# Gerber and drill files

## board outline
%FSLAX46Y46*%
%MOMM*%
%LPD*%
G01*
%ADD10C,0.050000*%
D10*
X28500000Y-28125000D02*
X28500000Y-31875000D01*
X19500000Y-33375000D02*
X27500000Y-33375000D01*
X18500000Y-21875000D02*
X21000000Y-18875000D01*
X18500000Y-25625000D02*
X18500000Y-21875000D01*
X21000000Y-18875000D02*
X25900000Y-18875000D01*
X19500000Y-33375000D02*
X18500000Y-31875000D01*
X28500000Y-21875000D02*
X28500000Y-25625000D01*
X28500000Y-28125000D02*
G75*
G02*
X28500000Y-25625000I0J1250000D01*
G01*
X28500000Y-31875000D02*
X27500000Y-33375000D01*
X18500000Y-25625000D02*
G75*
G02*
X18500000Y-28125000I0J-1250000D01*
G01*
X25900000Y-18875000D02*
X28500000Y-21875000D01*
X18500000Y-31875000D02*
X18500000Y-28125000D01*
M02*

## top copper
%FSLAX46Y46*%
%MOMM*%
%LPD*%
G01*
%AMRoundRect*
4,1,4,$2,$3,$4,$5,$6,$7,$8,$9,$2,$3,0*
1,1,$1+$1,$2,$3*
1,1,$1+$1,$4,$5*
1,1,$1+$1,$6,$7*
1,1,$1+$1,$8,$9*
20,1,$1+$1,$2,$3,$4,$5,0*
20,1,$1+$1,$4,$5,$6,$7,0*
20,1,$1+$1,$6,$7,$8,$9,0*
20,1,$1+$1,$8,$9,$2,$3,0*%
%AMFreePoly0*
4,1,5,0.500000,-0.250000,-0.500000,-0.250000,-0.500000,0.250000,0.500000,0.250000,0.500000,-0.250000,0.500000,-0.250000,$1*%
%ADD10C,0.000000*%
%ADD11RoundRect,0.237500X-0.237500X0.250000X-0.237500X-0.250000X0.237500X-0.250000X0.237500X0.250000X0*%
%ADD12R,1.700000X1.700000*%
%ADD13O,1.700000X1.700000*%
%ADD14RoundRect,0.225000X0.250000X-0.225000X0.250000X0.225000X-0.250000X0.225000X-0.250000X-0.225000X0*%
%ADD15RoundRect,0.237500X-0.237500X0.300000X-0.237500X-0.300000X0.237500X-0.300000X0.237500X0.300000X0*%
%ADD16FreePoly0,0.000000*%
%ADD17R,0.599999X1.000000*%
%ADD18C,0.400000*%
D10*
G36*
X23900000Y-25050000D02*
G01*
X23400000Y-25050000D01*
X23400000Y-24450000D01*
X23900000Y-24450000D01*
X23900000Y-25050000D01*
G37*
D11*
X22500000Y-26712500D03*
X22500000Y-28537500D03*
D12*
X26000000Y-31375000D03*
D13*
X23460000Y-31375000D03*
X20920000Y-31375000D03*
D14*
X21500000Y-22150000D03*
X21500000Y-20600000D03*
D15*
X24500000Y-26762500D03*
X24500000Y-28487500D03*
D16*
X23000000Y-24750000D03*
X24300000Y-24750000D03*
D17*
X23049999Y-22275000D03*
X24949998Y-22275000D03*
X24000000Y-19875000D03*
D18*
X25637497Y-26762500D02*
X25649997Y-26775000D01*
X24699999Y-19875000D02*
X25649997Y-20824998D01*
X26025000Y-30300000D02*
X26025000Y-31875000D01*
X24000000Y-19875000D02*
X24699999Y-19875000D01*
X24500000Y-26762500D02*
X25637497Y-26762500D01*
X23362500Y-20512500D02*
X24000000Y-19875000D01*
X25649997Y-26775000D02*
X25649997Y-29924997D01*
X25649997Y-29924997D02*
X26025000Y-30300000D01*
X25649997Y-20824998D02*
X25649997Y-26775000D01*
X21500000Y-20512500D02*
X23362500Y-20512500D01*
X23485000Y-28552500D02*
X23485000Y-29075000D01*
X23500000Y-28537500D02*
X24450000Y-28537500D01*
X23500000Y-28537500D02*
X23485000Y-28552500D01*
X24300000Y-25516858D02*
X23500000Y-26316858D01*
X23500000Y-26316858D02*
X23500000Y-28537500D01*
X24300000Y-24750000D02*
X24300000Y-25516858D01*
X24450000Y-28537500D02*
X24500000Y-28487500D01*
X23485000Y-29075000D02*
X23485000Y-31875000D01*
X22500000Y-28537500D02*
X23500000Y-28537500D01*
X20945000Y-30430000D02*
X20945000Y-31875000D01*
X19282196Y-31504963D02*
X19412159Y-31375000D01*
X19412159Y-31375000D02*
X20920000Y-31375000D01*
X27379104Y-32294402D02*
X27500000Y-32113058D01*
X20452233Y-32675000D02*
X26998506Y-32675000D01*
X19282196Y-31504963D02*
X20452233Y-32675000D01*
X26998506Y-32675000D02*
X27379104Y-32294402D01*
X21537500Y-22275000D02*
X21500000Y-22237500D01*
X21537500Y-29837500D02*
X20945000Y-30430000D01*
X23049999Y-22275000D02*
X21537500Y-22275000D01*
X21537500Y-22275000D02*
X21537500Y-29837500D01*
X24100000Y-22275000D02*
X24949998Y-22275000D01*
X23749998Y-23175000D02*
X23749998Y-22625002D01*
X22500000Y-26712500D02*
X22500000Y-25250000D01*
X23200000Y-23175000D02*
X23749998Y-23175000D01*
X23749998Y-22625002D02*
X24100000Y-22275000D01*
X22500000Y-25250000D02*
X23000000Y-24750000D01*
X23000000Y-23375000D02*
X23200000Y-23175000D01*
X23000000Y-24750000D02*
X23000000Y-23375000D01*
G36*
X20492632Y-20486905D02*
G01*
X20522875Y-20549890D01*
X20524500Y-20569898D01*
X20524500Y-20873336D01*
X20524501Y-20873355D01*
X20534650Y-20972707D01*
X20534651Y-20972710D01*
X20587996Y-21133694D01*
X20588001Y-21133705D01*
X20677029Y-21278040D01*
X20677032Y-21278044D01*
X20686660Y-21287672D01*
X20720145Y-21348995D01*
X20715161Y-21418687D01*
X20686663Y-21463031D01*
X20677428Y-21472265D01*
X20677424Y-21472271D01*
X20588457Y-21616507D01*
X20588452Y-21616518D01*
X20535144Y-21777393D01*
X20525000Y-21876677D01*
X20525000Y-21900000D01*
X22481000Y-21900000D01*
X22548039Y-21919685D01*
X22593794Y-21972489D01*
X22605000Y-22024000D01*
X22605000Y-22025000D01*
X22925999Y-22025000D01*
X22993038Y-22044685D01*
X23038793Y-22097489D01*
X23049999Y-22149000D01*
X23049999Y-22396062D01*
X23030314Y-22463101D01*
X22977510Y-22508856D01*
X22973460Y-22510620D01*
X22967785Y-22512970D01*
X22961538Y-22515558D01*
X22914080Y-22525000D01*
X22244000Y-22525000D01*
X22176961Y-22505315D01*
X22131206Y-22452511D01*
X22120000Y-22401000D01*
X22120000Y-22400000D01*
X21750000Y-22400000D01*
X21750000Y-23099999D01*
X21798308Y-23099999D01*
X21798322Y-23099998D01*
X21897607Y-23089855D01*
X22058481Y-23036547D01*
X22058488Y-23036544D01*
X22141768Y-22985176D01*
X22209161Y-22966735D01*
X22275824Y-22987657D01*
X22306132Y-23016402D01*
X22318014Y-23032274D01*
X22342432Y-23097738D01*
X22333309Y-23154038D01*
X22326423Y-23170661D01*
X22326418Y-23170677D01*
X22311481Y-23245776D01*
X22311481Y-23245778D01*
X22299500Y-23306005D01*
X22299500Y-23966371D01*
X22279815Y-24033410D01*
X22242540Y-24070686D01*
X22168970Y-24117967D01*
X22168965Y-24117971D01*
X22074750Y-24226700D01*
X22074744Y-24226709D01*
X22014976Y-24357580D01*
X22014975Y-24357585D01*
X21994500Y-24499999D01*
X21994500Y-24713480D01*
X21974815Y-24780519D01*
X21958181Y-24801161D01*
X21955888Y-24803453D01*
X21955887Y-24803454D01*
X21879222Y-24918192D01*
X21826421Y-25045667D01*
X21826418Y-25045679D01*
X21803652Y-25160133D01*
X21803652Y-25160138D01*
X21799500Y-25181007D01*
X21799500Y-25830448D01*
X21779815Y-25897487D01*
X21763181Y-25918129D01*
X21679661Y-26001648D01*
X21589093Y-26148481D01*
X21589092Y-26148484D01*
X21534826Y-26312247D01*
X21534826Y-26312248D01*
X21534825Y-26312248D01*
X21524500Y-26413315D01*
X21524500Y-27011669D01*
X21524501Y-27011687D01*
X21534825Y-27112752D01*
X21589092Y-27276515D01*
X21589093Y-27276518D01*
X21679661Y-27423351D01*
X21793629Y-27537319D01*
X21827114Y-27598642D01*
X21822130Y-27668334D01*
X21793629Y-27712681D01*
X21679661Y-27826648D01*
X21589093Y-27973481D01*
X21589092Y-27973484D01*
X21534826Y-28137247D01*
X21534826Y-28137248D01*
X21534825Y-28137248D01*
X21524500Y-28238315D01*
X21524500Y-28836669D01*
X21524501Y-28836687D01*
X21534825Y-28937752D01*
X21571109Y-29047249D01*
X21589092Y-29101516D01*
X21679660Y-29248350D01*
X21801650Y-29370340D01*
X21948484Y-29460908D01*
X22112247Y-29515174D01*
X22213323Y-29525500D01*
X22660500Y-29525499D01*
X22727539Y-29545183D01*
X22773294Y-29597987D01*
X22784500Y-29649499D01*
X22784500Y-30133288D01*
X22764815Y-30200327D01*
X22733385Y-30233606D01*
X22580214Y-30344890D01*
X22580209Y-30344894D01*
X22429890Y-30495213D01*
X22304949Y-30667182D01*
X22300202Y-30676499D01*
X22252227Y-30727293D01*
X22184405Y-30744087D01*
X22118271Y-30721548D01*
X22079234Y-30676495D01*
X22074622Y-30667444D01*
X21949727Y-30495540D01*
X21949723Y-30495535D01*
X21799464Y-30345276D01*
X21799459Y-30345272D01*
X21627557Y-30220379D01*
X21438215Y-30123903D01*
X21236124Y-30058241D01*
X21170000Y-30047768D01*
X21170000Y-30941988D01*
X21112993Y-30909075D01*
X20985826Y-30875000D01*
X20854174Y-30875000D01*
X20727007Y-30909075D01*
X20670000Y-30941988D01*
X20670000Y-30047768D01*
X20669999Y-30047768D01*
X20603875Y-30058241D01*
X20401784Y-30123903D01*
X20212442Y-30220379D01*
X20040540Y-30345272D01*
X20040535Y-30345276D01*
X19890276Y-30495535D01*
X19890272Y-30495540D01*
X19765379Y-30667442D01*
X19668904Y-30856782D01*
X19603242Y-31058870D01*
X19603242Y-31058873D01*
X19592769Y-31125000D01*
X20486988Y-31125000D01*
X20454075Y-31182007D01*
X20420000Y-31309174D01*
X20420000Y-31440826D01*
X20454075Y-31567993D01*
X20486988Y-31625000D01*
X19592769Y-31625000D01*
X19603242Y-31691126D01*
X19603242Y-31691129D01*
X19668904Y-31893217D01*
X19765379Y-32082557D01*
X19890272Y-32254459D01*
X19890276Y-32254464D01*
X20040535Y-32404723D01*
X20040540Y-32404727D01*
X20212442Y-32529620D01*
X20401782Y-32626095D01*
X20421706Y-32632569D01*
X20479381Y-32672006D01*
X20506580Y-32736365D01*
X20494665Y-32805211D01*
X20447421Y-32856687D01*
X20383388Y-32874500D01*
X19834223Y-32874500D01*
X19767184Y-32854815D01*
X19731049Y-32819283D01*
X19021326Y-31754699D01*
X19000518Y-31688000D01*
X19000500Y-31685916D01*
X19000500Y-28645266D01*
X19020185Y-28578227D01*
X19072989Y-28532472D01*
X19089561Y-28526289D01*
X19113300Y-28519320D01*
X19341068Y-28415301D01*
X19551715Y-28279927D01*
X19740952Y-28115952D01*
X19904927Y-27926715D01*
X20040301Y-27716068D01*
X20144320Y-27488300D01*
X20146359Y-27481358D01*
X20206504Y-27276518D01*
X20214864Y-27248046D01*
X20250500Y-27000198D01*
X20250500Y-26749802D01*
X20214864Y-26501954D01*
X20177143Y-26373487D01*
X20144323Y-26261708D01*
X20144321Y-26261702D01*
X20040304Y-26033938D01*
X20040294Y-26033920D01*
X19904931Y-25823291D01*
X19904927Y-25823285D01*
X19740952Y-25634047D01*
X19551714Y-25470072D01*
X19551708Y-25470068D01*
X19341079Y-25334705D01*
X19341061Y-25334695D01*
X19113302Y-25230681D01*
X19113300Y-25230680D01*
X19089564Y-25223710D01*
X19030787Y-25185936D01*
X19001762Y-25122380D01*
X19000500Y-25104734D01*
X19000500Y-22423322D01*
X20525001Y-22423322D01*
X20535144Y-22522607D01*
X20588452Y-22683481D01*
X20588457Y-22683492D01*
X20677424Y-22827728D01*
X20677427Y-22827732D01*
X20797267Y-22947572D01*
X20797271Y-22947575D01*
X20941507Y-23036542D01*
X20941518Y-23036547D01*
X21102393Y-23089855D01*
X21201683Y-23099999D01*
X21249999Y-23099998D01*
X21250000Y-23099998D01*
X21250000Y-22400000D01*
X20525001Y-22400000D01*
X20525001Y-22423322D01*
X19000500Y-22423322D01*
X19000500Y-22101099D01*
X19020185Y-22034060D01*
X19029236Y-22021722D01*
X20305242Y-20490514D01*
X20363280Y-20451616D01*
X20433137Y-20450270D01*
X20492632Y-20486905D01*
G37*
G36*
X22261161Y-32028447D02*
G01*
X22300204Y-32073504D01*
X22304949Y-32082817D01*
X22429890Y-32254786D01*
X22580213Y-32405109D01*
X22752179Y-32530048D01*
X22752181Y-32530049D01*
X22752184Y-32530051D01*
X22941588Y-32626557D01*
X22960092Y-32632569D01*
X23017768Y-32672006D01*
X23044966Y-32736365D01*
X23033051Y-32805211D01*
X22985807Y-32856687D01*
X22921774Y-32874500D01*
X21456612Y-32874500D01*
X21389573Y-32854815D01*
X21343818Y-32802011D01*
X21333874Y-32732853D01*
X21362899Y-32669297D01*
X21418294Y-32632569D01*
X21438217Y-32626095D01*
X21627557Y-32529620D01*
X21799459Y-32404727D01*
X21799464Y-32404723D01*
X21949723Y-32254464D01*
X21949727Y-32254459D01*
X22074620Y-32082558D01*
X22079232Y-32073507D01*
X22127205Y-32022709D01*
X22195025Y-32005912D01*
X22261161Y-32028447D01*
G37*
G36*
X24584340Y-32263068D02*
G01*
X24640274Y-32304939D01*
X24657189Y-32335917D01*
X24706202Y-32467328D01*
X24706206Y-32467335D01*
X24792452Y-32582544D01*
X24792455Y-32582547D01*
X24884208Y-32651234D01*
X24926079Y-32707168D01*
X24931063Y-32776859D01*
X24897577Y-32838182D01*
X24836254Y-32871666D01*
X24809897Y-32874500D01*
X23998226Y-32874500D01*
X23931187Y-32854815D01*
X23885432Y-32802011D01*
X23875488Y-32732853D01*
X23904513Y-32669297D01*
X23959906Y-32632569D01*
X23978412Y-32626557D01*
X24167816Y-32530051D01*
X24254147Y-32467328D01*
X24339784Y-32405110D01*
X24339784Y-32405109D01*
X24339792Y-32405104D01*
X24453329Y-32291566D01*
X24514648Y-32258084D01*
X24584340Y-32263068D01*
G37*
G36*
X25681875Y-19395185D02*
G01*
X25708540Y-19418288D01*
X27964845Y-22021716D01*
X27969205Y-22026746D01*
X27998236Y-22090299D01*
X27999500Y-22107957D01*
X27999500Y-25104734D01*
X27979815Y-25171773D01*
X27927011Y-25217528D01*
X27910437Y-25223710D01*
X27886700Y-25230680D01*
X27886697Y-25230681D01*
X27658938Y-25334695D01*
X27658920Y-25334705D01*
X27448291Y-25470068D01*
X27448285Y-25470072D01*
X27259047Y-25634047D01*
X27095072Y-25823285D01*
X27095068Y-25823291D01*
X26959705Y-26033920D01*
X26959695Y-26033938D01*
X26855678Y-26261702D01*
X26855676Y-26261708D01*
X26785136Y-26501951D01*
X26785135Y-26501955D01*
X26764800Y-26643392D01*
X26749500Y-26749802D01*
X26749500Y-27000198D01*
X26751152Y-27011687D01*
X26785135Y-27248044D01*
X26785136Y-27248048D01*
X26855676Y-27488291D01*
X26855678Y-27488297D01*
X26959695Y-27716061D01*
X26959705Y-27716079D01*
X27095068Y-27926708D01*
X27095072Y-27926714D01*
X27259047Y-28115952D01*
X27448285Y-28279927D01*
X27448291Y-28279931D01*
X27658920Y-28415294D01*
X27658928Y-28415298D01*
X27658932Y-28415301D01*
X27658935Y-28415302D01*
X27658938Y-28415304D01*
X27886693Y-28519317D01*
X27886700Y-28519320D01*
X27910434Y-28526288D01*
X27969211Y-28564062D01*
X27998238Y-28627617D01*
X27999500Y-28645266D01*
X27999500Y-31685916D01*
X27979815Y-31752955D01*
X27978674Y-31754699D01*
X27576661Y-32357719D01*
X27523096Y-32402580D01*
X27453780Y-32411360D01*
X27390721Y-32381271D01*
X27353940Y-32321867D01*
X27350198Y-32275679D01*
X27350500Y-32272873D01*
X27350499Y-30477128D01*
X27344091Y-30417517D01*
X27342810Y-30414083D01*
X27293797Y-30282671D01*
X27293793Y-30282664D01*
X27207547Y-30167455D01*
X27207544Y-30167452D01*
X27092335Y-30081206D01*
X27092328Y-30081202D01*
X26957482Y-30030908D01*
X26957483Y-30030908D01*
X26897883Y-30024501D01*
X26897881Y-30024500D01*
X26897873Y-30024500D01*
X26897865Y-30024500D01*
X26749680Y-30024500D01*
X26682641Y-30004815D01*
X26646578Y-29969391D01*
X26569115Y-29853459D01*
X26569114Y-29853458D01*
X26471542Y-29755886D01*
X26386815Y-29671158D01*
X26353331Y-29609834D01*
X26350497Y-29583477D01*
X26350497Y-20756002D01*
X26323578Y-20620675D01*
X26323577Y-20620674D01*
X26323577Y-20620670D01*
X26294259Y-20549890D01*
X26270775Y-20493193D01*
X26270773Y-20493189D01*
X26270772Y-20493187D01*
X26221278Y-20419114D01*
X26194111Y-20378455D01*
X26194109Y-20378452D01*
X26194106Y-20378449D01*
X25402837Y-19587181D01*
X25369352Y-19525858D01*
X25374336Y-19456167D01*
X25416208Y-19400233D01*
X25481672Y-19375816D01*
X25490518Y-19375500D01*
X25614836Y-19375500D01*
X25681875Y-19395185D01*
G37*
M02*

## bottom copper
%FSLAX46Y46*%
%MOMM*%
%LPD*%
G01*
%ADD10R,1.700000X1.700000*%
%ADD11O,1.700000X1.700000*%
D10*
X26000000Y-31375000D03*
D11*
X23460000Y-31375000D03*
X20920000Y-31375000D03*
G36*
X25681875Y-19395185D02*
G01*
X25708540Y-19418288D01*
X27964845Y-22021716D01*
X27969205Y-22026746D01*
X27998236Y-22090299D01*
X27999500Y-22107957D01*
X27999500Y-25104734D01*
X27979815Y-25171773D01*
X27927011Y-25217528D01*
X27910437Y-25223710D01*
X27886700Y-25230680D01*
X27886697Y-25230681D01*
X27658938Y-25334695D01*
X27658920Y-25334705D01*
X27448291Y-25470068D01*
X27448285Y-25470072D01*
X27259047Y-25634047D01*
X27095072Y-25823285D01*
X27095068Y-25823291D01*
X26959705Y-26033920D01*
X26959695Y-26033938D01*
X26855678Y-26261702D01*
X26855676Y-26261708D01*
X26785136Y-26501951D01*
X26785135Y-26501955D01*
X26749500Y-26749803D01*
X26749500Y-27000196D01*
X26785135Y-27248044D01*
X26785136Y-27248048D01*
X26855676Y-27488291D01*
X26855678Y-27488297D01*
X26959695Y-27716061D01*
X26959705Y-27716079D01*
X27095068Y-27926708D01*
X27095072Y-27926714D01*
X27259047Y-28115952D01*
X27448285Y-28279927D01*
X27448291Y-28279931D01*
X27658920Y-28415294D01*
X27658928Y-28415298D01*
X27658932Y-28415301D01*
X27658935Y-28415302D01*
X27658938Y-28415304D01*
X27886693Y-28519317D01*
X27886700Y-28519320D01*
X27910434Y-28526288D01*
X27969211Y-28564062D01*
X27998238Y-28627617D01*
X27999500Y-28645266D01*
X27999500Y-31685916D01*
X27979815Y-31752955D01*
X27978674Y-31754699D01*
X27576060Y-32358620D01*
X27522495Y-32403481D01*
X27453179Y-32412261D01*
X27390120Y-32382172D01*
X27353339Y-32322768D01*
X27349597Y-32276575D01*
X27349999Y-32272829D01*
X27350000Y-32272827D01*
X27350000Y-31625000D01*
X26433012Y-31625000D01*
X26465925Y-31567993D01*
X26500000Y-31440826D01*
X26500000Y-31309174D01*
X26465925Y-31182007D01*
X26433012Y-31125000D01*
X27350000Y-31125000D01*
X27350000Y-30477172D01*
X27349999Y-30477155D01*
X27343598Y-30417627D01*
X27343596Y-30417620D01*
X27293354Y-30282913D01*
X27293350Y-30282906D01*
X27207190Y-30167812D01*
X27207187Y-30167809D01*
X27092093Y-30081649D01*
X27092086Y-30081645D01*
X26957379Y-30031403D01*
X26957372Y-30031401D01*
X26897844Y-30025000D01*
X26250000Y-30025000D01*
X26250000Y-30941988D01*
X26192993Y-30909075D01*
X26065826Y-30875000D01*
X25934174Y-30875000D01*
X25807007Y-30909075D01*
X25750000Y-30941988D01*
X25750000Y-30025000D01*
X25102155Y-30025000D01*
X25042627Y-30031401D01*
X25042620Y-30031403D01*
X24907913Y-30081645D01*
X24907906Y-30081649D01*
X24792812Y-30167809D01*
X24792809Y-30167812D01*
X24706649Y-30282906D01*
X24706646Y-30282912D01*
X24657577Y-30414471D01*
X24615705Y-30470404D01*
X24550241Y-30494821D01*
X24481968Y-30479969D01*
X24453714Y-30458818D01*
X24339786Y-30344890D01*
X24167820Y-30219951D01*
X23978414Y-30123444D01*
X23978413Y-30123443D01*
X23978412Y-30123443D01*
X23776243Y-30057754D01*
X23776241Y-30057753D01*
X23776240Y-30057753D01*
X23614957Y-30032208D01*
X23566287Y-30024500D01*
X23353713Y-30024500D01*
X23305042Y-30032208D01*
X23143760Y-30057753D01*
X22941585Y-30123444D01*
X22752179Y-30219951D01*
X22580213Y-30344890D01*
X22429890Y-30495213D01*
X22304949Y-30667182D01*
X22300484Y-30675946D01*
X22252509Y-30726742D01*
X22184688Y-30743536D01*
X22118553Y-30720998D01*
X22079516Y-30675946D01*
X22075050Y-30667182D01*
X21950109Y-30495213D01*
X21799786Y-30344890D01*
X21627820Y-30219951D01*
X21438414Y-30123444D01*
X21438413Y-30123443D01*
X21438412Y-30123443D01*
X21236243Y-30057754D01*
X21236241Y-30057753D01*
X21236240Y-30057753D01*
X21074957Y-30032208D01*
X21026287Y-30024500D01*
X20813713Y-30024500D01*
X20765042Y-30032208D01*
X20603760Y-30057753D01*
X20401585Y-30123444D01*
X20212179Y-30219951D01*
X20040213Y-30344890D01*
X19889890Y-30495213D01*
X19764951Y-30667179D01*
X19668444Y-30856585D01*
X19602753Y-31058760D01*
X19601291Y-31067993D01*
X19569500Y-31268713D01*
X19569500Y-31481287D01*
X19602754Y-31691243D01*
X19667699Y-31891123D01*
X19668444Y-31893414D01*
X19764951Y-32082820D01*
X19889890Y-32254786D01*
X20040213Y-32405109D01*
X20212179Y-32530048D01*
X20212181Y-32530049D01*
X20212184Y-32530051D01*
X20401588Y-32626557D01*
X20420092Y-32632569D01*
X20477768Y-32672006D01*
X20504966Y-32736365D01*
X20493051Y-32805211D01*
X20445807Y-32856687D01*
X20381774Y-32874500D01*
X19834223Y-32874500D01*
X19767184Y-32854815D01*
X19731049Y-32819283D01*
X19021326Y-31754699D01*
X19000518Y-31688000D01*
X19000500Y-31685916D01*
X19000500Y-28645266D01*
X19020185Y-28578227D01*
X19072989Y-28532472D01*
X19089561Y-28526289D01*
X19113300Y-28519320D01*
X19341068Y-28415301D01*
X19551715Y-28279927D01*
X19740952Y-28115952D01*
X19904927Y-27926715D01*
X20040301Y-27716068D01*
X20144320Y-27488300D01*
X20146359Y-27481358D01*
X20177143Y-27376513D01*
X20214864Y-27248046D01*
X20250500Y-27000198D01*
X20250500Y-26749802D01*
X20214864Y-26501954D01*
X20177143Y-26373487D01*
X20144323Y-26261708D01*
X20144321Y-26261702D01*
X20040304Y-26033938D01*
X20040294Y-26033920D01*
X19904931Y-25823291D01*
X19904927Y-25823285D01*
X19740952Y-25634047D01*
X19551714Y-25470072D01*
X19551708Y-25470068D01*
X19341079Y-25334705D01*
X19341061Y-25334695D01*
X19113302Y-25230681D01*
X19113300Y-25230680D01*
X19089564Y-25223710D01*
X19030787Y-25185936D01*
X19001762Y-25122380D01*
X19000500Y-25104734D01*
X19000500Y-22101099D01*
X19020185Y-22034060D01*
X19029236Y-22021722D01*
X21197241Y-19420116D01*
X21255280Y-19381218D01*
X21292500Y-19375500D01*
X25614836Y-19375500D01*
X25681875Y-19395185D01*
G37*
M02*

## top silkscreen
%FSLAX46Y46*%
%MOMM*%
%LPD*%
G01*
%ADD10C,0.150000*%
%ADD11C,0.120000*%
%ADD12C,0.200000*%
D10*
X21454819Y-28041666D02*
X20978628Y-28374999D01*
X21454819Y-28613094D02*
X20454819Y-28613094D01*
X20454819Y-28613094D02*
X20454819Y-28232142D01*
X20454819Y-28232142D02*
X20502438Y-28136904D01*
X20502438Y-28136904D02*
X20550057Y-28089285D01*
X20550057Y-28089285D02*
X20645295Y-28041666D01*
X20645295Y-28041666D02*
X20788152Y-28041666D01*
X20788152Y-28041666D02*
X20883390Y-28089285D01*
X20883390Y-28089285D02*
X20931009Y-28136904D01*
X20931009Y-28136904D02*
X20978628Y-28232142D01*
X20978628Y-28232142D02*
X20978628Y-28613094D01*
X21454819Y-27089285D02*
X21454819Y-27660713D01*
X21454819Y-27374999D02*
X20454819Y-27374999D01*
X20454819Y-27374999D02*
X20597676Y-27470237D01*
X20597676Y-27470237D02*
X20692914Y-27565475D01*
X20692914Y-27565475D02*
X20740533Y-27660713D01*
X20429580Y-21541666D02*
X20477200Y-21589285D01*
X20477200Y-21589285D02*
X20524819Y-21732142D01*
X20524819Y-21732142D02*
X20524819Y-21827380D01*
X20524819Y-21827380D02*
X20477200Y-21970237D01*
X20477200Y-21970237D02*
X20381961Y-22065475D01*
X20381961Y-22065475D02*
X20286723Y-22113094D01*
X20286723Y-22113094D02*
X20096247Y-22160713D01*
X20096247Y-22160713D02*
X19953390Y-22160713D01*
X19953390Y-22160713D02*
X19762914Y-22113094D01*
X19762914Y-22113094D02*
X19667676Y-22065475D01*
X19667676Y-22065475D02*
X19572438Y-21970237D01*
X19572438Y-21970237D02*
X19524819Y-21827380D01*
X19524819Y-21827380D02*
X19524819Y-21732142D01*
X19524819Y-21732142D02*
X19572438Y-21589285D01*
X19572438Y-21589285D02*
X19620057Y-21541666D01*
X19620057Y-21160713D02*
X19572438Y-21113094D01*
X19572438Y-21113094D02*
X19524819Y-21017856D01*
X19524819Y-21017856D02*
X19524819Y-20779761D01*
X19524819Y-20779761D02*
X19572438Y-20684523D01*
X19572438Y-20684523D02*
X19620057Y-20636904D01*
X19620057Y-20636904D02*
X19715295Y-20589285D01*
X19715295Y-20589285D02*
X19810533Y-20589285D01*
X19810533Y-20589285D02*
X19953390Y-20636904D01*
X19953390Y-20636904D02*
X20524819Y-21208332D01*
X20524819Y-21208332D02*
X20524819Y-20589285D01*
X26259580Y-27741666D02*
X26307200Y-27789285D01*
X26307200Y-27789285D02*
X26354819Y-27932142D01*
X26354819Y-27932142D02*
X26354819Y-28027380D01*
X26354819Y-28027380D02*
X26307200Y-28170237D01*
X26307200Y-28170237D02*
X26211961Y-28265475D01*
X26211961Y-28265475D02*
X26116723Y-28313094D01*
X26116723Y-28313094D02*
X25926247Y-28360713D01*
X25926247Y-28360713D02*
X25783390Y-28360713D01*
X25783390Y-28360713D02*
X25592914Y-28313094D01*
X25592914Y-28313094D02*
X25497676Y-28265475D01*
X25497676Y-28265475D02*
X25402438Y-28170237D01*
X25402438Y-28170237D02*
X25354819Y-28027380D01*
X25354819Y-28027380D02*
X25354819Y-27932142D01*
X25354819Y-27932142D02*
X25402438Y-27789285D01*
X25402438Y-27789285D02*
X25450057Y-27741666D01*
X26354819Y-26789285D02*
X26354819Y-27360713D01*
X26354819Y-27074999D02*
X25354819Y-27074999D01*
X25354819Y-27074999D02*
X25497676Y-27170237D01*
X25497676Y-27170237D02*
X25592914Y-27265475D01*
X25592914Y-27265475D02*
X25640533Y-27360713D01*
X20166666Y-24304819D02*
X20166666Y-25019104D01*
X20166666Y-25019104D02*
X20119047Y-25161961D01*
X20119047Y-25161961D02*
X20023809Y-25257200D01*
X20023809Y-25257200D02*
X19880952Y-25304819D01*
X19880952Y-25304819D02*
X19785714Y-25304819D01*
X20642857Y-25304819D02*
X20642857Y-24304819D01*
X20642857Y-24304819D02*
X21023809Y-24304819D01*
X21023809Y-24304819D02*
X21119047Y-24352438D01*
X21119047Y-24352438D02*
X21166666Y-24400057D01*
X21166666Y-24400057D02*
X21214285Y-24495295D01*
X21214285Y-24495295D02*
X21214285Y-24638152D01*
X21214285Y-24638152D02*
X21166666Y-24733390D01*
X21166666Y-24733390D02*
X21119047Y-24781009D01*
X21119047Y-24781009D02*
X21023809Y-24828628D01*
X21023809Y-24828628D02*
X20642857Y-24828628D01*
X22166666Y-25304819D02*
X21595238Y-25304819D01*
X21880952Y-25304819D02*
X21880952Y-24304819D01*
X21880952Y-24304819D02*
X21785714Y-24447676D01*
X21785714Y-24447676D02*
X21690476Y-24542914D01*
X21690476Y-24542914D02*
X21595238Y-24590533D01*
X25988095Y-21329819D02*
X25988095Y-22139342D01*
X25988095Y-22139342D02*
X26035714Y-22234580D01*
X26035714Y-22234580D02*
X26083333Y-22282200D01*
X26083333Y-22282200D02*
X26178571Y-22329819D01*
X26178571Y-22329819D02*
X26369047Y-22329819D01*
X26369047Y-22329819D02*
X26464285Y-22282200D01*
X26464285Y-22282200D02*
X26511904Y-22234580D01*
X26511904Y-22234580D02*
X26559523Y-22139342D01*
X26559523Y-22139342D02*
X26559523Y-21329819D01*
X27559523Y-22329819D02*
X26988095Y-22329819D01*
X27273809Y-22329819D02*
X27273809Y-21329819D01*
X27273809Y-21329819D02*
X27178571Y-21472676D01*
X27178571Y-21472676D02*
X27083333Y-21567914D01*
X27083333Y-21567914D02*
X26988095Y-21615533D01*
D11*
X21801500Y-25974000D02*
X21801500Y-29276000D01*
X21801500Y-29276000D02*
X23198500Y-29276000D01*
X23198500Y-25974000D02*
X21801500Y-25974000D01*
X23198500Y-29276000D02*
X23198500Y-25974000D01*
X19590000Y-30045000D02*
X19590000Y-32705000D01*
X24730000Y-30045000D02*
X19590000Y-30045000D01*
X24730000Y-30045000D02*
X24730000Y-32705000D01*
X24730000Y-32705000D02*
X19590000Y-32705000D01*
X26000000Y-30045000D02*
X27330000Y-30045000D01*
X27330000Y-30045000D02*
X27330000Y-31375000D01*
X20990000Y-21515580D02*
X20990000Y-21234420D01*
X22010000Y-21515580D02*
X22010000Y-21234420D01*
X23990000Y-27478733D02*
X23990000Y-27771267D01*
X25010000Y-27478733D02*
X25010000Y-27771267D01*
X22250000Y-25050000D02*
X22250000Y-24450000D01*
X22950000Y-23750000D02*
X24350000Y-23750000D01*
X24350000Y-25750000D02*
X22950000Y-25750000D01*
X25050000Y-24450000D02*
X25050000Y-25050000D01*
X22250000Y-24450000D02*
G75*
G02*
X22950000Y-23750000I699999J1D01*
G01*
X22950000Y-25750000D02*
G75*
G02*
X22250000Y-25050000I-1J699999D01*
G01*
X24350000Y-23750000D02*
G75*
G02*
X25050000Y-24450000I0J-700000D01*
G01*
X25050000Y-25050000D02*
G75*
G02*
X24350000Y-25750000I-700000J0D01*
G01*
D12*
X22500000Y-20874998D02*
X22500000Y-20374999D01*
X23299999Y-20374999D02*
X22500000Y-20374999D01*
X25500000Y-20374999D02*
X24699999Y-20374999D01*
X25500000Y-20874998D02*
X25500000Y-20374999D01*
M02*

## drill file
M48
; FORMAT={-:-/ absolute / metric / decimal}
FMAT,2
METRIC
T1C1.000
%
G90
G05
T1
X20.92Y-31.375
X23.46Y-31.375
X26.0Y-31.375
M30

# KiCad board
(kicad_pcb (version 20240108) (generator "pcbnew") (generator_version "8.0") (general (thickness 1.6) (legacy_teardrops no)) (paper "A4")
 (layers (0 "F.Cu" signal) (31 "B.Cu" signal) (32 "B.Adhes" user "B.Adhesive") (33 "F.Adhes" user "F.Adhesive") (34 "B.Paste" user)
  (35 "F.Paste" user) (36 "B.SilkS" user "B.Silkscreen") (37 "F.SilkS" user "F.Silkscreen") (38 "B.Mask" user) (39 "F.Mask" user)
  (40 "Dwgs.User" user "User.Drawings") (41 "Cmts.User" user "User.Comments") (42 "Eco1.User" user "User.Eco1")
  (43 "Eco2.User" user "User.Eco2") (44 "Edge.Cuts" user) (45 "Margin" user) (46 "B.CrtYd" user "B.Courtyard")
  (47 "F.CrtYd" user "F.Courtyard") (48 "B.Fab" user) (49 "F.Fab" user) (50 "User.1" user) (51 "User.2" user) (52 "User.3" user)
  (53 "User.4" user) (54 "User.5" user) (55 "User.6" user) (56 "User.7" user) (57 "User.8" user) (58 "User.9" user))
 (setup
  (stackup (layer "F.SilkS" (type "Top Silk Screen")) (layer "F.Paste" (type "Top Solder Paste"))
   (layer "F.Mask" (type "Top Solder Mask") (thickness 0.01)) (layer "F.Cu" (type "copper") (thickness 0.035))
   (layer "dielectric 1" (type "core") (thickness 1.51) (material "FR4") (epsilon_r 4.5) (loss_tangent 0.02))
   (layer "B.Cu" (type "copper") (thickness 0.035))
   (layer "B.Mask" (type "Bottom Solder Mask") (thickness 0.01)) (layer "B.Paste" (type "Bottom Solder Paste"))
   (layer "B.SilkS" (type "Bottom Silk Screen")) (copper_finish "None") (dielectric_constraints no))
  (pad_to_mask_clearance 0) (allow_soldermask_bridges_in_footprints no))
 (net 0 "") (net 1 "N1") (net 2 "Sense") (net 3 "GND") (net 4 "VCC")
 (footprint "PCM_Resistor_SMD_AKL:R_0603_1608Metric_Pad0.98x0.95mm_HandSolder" (layer "F.Cu") (at 22.5 27.625 -90)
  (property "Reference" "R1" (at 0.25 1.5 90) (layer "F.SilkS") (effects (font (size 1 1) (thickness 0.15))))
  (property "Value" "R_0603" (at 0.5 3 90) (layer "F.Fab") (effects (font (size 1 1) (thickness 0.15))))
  (fp_line (start -1.651 0.6985) (end 1.651 0.6985) (stroke (width 0.12) (type solid)) (layer "F.SilkS"))
  (fp_line (start 1.651 0.6985) (end 1.651 -0.6985) (stroke (width 0.12) (type solid)) (layer "F.SilkS"))
  (fp_line (start -1.651 -0.6985) (end -1.651 0.6985) (stroke (width 0.12) (type solid)) (layer "F.SilkS"))
  (fp_line (start 1.651 -0.6985) (end -1.651 -0.6985) (stroke (width 0.12) (type solid)) (layer "F.SilkS"))
  (pad "1" smd roundrect (at -0.9125 0 270) (size 0.975 0.95) (layers "F.Cu" "F.Paste" "F.Mask") (roundrect_rratio 0.25) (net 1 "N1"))
  (pad "2" smd roundrect (at 0.9125 0 270) (size 0.975 0.95) (layers "F.Cu" "F.Paste" "F.Mask") (roundrect_rratio 0.25) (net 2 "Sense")))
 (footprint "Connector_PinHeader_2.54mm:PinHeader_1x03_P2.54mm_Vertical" (layer "F.Cu") (at 26 31.375 -90)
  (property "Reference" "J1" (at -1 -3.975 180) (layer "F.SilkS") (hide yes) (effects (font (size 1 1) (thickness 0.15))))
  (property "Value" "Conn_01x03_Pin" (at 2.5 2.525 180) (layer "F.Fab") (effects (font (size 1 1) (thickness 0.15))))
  (fp_line (start -1.33 6.41) (end 1.33 6.41) (stroke (width 0.12) (type solid)) (layer "F.SilkS"))
  (fp_line (start -1.33 1.27) (end -1.33 6.41) (stroke (width 0.12) (type solid)) (layer "F.SilkS"))
  (fp_line (start -1.33 1.27) (end 1.33 1.27) (stroke (width 0.12) (type solid)) (layer "F.SilkS"))
  (fp_line (start 1.33 1.27) (end 1.33 6.41) (stroke (width 0.12) (type solid)) (layer "F.SilkS"))
  (fp_line (start -1.33 0) (end -1.33 -1.33) (stroke (width 0.12) (type solid)) (layer "F.SilkS"))
  (fp_line (start -1.33 -1.33) (end 0 -1.33) (stroke (width 0.12) (type solid)) (layer "F.SilkS"))
  (pad "1" thru_hole rect (at 0 0 270) (size 1.7 1.7) (drill 1) (layers "*.Cu" "*.Mask") (remove_unused_layers no) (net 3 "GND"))
  (pad "2" thru_hole oval (at 0 2.54 270) (size 1.7 1.7) (drill 1) (layers "*.Cu" "*.Mask") (remove_unused_layers no) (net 2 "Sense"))
  (pad "3" thru_hole oval (at 0 5.08 270) (size 1.7 1.7) (drill 1) (layers "*.Cu" "*.Mask") (remove_unused_layers no) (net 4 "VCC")))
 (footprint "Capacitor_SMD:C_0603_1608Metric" (layer "F.Cu") (at 21.5 21.375 90)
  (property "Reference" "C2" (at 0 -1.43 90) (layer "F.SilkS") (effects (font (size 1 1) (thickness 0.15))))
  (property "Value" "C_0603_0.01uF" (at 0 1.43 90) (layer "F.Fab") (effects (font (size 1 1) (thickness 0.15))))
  (fp_line (start -0.14058 -0.51) (end 0.14058 -0.51) (stroke (width 0.12) (type solid)) (layer "F.SilkS"))
  (fp_line (start -0.14058 0.51) (end 0.14058 0.51) (stroke (width 0.12) (type solid)) (layer "F.SilkS"))
  (pad "1" smd roundrect (at -0.775 0 90) (size 0.9 0.95) (layers "F.Cu" "F.Paste" "F.Mask") (roundrect_rratio 0.25) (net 4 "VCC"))
  (pad "2" smd roundrect (at 0.775 0 90) (size 0.9 0.95) (layers "F.Cu" "F.Paste" "F.Mask") (roundrect_rratio 0.25) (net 3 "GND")))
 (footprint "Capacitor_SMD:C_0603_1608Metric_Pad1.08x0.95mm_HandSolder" (layer "F.Cu") (at 24.5 27.625 -90)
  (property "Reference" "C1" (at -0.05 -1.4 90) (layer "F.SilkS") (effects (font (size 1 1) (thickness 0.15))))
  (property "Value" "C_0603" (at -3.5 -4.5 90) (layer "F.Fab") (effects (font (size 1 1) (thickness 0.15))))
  (fp_line (start -0.146267 0.51) (end 0.146267 0.51) (stroke (width 0.12) (type solid)) (layer "F.SilkS"))
  (fp_line (start -0.146267 -0.51) (end 0.146267 -0.51) (stroke (width 0.12) (type solid)) (layer "F.SilkS"))
  (pad "1" smd roundrect (at -0.8625 0 270) (size 1.075 0.95) (layers "F.Cu" "F.Paste" "F.Mask") (roundrect_rratio 0.25) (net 3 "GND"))
  (pad "2" smd roundrect (at 0.8625 0 270) (size 1.075 0.95) (layers "F.Cu" "F.Paste" "F.Mask") (roundrect_rratio 0.25) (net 2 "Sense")))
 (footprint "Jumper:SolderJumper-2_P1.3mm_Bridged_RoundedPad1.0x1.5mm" (layer "F.Cu") (at 23.65 24.75)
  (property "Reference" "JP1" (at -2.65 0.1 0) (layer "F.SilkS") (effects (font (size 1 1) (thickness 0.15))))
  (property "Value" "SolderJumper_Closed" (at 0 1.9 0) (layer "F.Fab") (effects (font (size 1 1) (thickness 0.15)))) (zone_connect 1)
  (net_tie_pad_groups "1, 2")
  (fp_poly (pts (xy 0.25 -0.3) (xy -0.25 -0.3) (xy -0.25 0.3) (xy 0.25 0.3)) (stroke (width 0) (type solid)) (fill solid) (layer "F.Cu"))
  (fp_line (start -1.4 0.3) (end -1.4 -0.3) (stroke (width 0.12) (type solid)) (layer "F.SilkS"))
  (fp_line (start -0.7 -1) (end 0.7 -1) (stroke (width 0.12) (type solid)) (layer "F.SilkS"))
  (fp_line (start 0.7 1) (end -0.7 1) (stroke (width 0.12) (type solid)) (layer "F.SilkS"))
  (fp_line (start 1.4 -0.3) (end 1.4 0.3) (stroke (width 0.12) (type solid)) (layer "F.SilkS"))
  (fp_arc (start -1.4 -0.3) (mid -1.194975 -0.794975) (end -0.7 -1) (stroke (width 0.12) (type solid)) (layer "F.SilkS"))
  (fp_arc (start -0.7 1) (mid -1.194975 0.794975) (end -1.4 0.3) (stroke (width 0.12) (type solid)) (layer "F.SilkS"))
  (fp_arc (start 0.7 -1) (mid 1.194975 -0.794975) (end 1.4 -0.3) (stroke (width 0.12) (type solid)) (layer "F.SilkS"))
  (fp_arc (start 1.4 0.3) (mid 1.194975 0.794975) (end 0.7 1) (stroke (width 0.12) (type solid)) (layer "F.SilkS"))
  (pad "1" smd custom (at -0.65 0) (size 1 0.5) (layers "F.Cu" "F.Mask") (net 1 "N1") (zone_connect 2) (thermal_bridge_angle 45)
   (options (clearance outline) (anchor rect)) (primitives))
  (pad "2" smd custom (at 0.65 0) (size 1 0.5) (layers "F.Cu" "F.Mask") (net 2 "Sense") (zone_connect 2) (thermal_bridge_angle 45)
   (options (clearance outline) (anchor rect)) (primitives)))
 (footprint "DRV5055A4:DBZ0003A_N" (layer "F.Cu") (at 24 21.075 -90)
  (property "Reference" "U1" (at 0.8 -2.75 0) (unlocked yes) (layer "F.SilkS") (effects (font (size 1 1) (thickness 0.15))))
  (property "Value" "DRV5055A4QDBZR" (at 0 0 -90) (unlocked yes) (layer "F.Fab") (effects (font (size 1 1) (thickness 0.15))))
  (fp_line (start -0.200002 1.5) (end -0.700001 1.5) (stroke (width 0.2) (type solid)) (layer "F.SilkS"))
  (fp_line (start -0.700001 0.700001) (end -0.700001 1.5) (stroke (width 0.2) (type solid)) (layer "F.SilkS"))
  (fp_line (start -0.700001 -1.5) (end -0.700001 -0.699999) (stroke (width 0.2) (type solid)) (layer "F.SilkS"))
  (fp_line (start -0.200002 -1.5) (end -0.700001 -1.5) (stroke (width 0.2) (type solid)) (layer "F.SilkS"))
  (pad "1" smd rect (at 1.2 0.950001 180) (size 0.599999 1) (layers "F.Cu" "F.Paste" "F.Mask") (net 4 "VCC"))
  (pad "2" smd rect (at 1.2 -0.949998 180) (size 0.599999 1) (layers "F.Cu" "F.Paste" "F.Mask") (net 1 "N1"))
  (pad "3" smd rect (at -1.2 0 180) (size 0.599999 1) (layers "F.Cu" "F.Paste" "F.Mask") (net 3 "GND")))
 (gr_line (start 28.5 28.125) (end 28.5 31.875) (stroke (width 0.05) (type default)) (layer "Edge.Cuts"))
 (gr_line (start 19.5 33.375) (end 27.5 33.375) (stroke (width 0.05) (type default)) (layer "Edge.Cuts"))
 (gr_line (start 18.5 21.875) (end 21 18.875) (stroke (width 0.05) (type default)) (layer "Edge.Cuts"))
 (gr_line (start 18.5 25.625) (end 18.5 21.875) (stroke (width 0.05) (type default)) (layer "Edge.Cuts"))
 (gr_line (start 21 18.875) (end 25.9 18.875) (stroke (width 0.05) (type default)) (layer "Edge.Cuts"))
 (gr_line (start 19.5 33.375) (end 18.5 31.875) (stroke (width 0.05) (type default)) (layer "Edge.Cuts"))
 (gr_line (start 28.5 21.875) (end 28.5 25.625) (stroke (width 0.05) (type default)) (layer "Edge.Cuts"))
 (gr_arc (start 28.5 28.125) (mid 27.25 26.875) (end 28.5 25.625) (stroke (width 0.05) (type default)) (layer "Edge.Cuts"))
 (gr_line (start 28.5 31.875) (end 27.5 33.375) (stroke (width 0.05) (type default)) (layer "Edge.Cuts"))
 (gr_arc (start 18.5 25.625) (mid 19.75 26.875) (end 18.5 28.125) (stroke (width 0.05) (type default)) (layer "Edge.Cuts"))
 (gr_line (start 25.9 18.875) (end 28.5 21.875) (stroke (width 0.05) (type default)) (layer "Edge.Cuts"))
 (gr_line (start 18.5 31.875) (end 18.5 28.125) (stroke (width 0.05) (type default)) (layer "Edge.Cuts"))
 (segment (start 25.637497 26.7625) (end 25.649997 26.775) (width 0.4) (layer "F.Cu") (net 3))
 (segment (start 24.699999 19.875) (end 25.649997 20.824998) (width 0.4) (layer "F.Cu") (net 3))
 (segment (start 26.025 30.3) (end 26.025 31.875) (width 0.4) (layer "F.Cu") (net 3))
 (segment (start 24 19.875) (end 24.699999 19.875) (width 0.4) (layer "F.Cu") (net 3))
 (segment (start 24.5 26.7625) (end 25.637497 26.7625) (width 0.4) (layer "F.Cu") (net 3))
 (segment (start 23.3625 20.5125) (end 24 19.875) (width 0.4) (layer "F.Cu") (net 3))
 (segment (start 25.649997 26.775) (end 25.649997 29.924997) (width 0.4) (layer "F.Cu") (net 3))
 (segment (start 25.649997 29.924997) (end 26.025 30.3) (width 0.4) (layer "F.Cu") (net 3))
 (segment (start 25.649997 20.824998) (end 25.649997 26.775) (width 0.4) (layer "F.Cu") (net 3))
 (segment (start 21.5 20.5125) (end 23.3625 20.5125) (width 0.4) (layer "F.Cu") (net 3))
 (segment (start 23.485 28.5525) (end 23.485 29.075) (width 0.4) (layer "F.Cu") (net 2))
 (segment (start 23.5 28.5375) (end 24.45 28.5375) (width 0.4) (layer "F.Cu") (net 2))
 (segment (start 23.5 28.5375) (end 23.485 28.5525) (width 0.4) (layer "F.Cu") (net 2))
 (segment (start 24.3 25.516858) (end 23.5 26.316858) (width 0.4) (layer "F.Cu") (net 2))
 (segment (start 23.5 26.316858) (end 23.5 28.5375) (width 0.4) (layer "F.Cu") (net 2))
 (segment (start 24.3 24.75) (end 24.3 25.516858) (width 0.4) (layer "F.Cu") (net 2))
 (segment (start 24.45 28.5375) (end 24.5 28.4875) (width 0.4) (layer "F.Cu") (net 2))
 (segment (start 23.485 29.075) (end 23.485 31.875) (width 0.4) (layer "F.Cu") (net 2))
 (segment (start 22.5 28.5375) (end 23.5 28.5375) (width 0.4) (layer "F.Cu") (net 2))
 (segment (start 20.945 30.43) (end 20.945 31.875) (width 0.4) (layer "F.Cu") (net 4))
 (segment (start 19.282196 31.504963) (end 19.412159 31.375) (width 0.4) (layer "F.Cu") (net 4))
 (segment (start 19.412159 31.375) (end 20.92 31.375) (width 0.4) (layer "F.Cu") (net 4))
 (segment (start 27.379104 32.294402) (end 27.5 32.113058) (width 0.4) (layer "F.Cu") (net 4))
 (segment (start 20.452233 32.675) (end 26.998506 32.675) (width 0.4) (layer "F.Cu") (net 4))
 (segment (start 19.282196 31.504963) (end 20.452233 32.675) (width 0.4) (layer "F.Cu") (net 4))
 (segment (start 26.998506 32.675) (end 27.379104 32.294402) (width 0.4) (layer "F.Cu") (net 4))
 (segment (start 21.5375 22.275) (end 21.5 22.2375) (width 0.4) (layer "F.Cu") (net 4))
 (segment (start 21.5375 29.8375) (end 20.945 30.43) (width 0.4) (layer "F.Cu") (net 4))
 (segment (start 23.049999 22.275) (end 21.5375 22.275) (width 0.4) (layer "F.Cu") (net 4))
 (segment (start 21.5375 22.275) (end 21.5375 29.8375) (width 0.4) (layer "F.Cu") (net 4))
 (segment (start 24.1 22.275) (end 24.949998 22.275) (width 0.4) (layer "F.Cu") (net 1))
 (segment (start 23.749998 23.175) (end 23.749998 22.625002) (width 0.4) (layer "F.Cu") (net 1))
 (segment (start 22.5 26.7125) (end 22.5 25.25) (width 0.4) (layer "F.Cu") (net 1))
 (segment (start 23.2 23.175) (end 23.749998 23.175) (width 0.4) (layer "F.Cu") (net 1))
 (segment (start 23.749998 22.625002) (end 24.1 22.275) (width 0.4) (layer "F.Cu") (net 1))
 (segment (start 22.5 25.25) (end 23 24.75) (width 0.4) (layer "F.Cu") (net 1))
 (segment (start 23 23.375) (end 23.2 23.175) (width 0.4) (layer "F.Cu") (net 1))
 (segment (start 23 24.75) (end 23 23.375) (width 0.4) (layer "F.Cu") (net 1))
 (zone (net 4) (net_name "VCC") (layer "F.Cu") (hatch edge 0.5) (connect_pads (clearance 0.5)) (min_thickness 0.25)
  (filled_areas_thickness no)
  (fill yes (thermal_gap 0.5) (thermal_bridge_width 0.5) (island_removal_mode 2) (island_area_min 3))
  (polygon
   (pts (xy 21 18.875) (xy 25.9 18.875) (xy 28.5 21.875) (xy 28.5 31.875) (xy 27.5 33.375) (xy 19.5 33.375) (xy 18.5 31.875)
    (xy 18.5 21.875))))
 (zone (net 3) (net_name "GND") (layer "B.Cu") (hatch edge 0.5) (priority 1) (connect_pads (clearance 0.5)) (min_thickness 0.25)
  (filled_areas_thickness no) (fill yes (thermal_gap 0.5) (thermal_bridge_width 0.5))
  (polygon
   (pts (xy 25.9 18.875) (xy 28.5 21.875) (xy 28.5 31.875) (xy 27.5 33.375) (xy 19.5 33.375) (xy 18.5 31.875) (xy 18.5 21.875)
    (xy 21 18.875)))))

